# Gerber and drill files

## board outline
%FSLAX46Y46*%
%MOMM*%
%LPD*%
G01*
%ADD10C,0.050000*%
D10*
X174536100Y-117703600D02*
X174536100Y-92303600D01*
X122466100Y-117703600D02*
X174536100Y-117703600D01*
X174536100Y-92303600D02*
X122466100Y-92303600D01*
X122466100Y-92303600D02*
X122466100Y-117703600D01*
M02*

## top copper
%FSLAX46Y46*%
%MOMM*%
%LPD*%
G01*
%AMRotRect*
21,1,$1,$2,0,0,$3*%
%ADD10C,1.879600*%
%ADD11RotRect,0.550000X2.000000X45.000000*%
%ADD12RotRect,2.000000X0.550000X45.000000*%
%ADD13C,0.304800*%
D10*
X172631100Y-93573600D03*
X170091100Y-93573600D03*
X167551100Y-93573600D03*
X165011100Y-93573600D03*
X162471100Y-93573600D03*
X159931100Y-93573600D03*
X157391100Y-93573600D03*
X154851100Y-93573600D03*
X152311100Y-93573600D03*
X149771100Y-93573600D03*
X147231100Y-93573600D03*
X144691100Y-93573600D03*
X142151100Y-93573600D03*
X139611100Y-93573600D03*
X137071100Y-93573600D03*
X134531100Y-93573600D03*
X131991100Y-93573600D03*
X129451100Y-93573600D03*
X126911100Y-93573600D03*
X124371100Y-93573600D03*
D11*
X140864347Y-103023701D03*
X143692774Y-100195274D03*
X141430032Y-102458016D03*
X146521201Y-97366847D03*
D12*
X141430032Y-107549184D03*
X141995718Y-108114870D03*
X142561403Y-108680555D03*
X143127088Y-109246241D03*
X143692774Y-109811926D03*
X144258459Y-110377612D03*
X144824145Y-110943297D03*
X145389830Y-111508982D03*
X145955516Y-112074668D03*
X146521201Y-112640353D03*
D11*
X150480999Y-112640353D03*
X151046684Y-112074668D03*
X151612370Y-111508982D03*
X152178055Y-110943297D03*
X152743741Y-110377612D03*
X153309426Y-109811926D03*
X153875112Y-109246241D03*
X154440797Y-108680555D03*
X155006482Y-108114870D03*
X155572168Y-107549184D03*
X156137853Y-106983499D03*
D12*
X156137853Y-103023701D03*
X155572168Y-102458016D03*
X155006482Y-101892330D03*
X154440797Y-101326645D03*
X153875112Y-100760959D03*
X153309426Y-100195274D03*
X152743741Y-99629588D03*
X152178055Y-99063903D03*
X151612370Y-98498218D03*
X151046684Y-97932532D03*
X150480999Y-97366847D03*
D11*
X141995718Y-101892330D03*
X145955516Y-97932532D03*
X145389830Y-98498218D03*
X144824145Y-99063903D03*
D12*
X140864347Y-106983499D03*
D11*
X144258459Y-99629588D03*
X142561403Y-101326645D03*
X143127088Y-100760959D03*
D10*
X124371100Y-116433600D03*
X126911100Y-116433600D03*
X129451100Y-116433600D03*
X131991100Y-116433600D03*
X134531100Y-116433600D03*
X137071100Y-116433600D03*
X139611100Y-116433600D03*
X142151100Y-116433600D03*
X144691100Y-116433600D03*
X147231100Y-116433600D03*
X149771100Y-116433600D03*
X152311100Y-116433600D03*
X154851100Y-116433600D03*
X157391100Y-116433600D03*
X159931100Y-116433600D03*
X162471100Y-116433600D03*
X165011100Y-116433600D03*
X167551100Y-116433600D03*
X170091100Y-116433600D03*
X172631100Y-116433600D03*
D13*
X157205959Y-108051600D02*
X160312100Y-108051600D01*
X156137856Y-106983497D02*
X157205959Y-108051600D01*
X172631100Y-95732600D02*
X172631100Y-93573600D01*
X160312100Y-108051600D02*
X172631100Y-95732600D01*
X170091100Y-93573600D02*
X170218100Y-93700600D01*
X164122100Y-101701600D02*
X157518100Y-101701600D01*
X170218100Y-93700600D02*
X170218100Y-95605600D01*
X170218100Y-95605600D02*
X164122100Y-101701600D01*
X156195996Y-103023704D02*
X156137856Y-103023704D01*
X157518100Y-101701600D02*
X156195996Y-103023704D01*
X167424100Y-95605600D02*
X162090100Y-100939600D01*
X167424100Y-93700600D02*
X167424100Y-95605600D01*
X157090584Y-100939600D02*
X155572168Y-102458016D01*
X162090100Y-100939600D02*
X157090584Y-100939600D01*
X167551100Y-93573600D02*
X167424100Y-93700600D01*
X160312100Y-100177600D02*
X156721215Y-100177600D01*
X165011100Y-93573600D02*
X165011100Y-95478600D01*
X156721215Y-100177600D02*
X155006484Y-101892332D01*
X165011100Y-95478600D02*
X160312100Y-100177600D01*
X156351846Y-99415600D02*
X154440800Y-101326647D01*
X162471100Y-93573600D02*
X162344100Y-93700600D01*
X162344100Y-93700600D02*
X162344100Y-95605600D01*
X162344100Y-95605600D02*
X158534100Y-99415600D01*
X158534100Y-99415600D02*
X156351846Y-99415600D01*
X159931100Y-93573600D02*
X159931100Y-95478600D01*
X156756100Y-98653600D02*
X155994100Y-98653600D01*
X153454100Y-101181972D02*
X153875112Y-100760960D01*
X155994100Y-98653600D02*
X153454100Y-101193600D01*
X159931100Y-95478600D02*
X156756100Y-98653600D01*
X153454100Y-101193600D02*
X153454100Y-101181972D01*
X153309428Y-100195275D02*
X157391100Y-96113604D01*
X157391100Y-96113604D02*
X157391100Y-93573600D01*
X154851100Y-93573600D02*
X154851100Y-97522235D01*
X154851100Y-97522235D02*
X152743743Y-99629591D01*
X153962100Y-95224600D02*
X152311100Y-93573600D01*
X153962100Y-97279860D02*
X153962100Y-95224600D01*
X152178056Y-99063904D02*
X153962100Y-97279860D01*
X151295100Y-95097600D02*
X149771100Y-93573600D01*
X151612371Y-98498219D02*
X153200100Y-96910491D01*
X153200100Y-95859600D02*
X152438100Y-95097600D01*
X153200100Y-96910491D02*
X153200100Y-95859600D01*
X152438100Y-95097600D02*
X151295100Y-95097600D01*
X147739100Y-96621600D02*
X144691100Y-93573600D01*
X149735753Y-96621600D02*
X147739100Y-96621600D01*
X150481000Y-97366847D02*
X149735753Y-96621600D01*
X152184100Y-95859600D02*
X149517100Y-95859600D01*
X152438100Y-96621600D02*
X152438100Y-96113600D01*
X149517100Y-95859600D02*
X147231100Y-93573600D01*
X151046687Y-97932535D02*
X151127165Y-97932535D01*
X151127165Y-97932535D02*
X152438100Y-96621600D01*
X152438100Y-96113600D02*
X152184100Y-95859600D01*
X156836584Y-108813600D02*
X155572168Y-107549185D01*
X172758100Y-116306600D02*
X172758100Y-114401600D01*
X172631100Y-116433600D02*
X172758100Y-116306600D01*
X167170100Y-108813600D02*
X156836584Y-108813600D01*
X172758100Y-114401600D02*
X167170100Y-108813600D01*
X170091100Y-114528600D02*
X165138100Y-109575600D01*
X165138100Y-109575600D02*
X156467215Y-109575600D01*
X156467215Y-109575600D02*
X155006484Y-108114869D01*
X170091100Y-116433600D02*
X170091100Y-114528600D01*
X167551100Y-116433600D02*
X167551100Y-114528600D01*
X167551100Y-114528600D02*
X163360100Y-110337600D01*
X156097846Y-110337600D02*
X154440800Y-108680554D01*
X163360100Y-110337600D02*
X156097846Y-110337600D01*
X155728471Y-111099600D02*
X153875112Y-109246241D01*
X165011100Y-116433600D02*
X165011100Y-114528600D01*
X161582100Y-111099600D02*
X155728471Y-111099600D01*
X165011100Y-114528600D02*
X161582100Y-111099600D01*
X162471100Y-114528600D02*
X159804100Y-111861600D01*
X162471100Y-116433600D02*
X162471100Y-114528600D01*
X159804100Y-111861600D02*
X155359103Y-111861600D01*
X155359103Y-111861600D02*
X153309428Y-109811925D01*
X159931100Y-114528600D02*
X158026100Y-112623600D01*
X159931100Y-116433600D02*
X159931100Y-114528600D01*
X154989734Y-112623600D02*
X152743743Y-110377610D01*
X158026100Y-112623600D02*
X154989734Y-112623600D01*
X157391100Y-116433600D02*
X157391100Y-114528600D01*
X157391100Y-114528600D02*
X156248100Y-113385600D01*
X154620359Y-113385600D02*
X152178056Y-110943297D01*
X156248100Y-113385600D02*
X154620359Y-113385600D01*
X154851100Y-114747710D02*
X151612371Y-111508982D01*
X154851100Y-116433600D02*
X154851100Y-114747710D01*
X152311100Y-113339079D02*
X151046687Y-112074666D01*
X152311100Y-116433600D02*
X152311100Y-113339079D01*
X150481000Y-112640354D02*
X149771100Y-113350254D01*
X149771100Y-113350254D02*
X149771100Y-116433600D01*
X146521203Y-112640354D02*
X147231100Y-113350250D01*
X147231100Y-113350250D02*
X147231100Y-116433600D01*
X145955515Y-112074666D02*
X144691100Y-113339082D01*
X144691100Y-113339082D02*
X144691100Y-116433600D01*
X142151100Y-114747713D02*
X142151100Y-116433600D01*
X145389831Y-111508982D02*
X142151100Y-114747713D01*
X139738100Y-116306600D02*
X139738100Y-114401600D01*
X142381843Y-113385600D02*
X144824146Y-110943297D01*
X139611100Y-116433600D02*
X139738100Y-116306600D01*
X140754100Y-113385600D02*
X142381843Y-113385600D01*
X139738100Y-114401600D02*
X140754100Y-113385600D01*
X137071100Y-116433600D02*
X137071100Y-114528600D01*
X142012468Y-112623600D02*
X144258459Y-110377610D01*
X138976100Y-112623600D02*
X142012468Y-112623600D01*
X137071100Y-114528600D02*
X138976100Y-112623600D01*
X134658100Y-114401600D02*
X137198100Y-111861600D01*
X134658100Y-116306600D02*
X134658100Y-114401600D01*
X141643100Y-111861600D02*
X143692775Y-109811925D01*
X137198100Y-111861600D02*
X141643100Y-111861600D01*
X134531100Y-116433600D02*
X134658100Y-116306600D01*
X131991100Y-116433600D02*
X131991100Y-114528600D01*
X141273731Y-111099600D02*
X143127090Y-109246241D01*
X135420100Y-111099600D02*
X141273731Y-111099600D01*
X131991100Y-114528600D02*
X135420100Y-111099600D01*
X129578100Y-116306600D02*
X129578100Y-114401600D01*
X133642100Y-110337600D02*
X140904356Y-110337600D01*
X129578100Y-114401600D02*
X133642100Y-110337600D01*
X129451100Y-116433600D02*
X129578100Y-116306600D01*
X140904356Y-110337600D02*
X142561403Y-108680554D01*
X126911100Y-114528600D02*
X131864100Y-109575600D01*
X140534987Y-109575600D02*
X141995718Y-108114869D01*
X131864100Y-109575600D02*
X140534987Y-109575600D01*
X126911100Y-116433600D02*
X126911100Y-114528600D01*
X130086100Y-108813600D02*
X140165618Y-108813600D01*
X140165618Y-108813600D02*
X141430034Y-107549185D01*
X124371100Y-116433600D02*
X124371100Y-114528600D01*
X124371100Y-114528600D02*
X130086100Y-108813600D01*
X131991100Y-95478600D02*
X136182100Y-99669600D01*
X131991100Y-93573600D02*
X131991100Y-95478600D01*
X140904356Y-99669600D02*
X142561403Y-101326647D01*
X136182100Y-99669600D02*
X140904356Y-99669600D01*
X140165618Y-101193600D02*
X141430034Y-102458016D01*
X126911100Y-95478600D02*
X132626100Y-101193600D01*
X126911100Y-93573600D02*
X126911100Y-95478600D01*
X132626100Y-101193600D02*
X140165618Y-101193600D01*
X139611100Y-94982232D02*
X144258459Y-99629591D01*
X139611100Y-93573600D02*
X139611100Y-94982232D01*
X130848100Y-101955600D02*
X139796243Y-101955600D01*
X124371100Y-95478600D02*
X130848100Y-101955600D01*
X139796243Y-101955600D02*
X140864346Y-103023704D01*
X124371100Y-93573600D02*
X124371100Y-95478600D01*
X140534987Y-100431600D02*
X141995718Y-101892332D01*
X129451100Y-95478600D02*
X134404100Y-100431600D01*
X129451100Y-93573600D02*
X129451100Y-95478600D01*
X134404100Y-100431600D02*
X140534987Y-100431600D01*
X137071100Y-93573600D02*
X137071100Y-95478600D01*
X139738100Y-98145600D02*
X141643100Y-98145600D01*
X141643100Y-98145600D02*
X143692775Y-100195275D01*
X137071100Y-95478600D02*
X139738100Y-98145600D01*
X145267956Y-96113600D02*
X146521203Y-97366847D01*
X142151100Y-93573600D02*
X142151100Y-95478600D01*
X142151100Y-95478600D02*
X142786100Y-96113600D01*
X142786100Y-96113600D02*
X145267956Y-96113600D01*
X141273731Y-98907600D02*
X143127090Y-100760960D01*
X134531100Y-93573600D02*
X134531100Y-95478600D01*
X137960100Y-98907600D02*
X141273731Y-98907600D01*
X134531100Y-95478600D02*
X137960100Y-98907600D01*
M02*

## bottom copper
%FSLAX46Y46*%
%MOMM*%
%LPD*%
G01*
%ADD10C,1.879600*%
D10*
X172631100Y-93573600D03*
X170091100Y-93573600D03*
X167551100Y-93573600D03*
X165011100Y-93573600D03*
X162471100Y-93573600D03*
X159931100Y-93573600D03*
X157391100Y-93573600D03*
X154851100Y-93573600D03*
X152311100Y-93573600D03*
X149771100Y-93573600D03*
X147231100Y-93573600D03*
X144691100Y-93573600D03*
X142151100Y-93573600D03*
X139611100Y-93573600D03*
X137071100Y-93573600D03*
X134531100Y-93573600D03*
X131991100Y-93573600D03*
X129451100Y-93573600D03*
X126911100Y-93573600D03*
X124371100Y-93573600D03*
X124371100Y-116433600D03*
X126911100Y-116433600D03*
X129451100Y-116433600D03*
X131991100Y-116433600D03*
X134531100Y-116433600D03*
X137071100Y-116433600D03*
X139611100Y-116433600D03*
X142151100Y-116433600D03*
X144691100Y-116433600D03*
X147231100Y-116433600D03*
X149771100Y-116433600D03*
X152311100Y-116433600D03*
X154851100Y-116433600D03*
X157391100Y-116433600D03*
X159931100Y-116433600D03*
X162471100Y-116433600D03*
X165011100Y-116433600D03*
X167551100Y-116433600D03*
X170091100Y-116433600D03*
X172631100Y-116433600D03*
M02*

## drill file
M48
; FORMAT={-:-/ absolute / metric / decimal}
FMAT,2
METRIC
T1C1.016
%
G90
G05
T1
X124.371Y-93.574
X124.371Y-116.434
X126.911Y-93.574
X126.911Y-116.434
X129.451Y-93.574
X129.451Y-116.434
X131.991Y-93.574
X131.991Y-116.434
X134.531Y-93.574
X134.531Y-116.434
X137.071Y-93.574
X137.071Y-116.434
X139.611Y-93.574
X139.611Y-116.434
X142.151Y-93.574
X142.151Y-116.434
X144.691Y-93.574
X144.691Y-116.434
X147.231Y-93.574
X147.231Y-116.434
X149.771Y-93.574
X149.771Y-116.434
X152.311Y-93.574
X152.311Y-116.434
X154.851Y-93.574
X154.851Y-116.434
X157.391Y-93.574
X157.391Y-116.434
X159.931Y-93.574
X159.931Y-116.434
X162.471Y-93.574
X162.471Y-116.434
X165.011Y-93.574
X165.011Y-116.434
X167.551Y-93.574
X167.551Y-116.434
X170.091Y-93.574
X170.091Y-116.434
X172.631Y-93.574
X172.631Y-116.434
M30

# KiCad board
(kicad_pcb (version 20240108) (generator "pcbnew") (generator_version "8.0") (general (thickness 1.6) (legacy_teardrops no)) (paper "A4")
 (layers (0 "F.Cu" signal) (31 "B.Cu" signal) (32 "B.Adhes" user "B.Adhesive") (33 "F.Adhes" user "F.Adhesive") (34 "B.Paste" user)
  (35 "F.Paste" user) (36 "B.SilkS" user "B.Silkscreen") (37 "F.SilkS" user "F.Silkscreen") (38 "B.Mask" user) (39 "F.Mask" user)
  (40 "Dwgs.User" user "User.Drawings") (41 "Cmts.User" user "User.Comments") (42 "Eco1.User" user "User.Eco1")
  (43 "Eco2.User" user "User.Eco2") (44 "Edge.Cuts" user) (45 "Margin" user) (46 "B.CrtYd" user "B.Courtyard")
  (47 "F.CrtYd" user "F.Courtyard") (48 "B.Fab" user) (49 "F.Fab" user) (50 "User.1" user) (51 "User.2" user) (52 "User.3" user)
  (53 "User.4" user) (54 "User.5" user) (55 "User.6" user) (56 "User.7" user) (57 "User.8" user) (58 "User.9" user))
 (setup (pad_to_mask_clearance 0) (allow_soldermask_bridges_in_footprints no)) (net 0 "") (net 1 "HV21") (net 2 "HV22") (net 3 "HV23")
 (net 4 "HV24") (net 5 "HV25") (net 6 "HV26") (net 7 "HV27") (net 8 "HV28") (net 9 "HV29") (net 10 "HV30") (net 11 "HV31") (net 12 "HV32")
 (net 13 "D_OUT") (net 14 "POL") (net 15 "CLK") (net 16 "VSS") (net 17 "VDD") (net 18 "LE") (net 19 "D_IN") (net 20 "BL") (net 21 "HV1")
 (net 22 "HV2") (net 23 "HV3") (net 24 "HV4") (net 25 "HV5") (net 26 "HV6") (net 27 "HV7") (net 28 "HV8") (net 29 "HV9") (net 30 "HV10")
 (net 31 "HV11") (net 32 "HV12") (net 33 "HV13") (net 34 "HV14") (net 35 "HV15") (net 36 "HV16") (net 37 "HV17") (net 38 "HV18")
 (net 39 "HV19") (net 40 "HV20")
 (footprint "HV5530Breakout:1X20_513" (layer "F.Cu") (at 172.6311 93.5736 180)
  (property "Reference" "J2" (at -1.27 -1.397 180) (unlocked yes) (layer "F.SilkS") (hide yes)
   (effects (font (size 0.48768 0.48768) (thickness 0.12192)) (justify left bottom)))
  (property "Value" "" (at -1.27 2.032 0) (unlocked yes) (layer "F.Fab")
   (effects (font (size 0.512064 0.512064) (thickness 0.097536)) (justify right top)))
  (pad "1" thru_hole circle (at 0 0 270) (size 1.8796 1.8796) (drill 1.016) (layers "*.Cu" "*.Mask") (remove_unused_layers no)
   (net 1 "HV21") (solder_mask_margin 0.1016) (thermal_bridge_angle 0))
  (pad "2" thru_hole circle (at 2.54 0 270) (size 1.8796 1.8796) (drill 1.016) (layers "*.Cu" "*.Mask") (remove_unused_layers no)
   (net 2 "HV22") (solder_mask_margin 0.1016) (thermal_bridge_angle 0))
  (pad "3" thru_hole circle (at 5.08 0 270) (size 1.8796 1.8796) (drill 1.016) (layers "*.Cu" "*.Mask") (remove_unused_layers no)
   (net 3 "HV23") (solder_mask_margin 0.1016) (thermal_bridge_angle 0))
  (pad "4" thru_hole circle (at 7.62 0 270) (size 1.8796 1.8796) (drill 1.016) (layers "*.Cu" "*.Mask") (remove_unused_layers no)
   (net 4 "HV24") (solder_mask_margin 0.1016) (thermal_bridge_angle 0))
  (pad "5" thru_hole circle (at 10.16 0 270) (size 1.8796 1.8796) (drill 1.016) (layers "*.Cu" "*.Mask") (remove_unused_layers no)
   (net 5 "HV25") (solder_mask_margin 0.1016) (thermal_bridge_angle 0))
  (pad "6" thru_hole circle (at 12.7 0 270) (size 1.8796 1.8796) (drill 1.016) (layers "*.Cu" "*.Mask") (remove_unused_layers no)
   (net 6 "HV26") (solder_mask_margin 0.1016) (thermal_bridge_angle 0))
  (pad "7" thru_hole circle (at 15.24 0 270) (size 1.8796 1.8796) (drill 1.016) (layers "*.Cu" "*.Mask") (remove_unused_layers no)
   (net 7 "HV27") (solder_mask_margin 0.1016) (thermal_bridge_angle 0))
  (pad "8" thru_hole circle (at 17.78 0 270) (size 1.8796 1.8796) (drill 1.016) (layers "*.Cu" "*.Mask") (remove_unused_layers no)
   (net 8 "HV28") (solder_mask_margin 0.1016) (thermal_bridge_angle 0))
  (pad "9" thru_hole circle (at 20.32 0 270) (size 1.8796 1.8796) (drill 1.016) (layers "*.Cu" "*.Mask") (remove_unused_layers no)
   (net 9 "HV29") (solder_mask_margin 0.1016) (thermal_bridge_angle 0))
  (pad "10" thru_hole circle (at 22.86 0 270) (size 1.8796 1.8796) (drill 1.016) (layers "*.Cu" "*.Mask") (remove_unused_layers no)
   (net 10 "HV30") (solder_mask_margin 0.1016) (thermal_bridge_angle 0))
  (pad "11" thru_hole circle (at 25.4 0 270) (size 1.8796 1.8796) (drill 1.016) (layers "*.Cu" "*.Mask") (remove_unused_layers no)
   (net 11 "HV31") (solder_mask_margin 0.1016) (thermal_bridge_angle 0))
  (pad "12" thru_hole circle (at 27.94 0 270) (size 1.8796 1.8796) (drill 1.016) (layers "*.Cu" "*.Mask") (remove_unused_layers no)
   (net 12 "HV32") (solder_mask_margin 0.1016) (thermal_bridge_angle 0))
  (pad "13" thru_hole circle (at 30.48 0 270) (size 1.8796 1.8796) (drill 1.016) (layers "*.Cu" "*.Mask") (remove_unused_layers no)
   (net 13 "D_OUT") (solder_mask_margin 0.1016) (thermal_bridge_angle 0))
  (pad "14" thru_hole circle (at 33.02 0 270) (size 1.8796 1.8796) (drill 1.016) (layers "*.Cu" "*.Mask") (remove_unused_layers no)
   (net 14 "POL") (solder_mask_margin 0.1016) (thermal_bridge_angle 0))
  (pad "15" thru_hole circle (at 35.56 0 270) (size 1.8796 1.8796) (drill 1.016) (layers "*.Cu" "*.Mask") (remove_unused_layers no)
   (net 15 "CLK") (solder_mask_margin 0.1016) (thermal_bridge_angle 0))
  (pad "16" thru_hole circle (at 38.1 0 270) (size 1.8796 1.8796) (drill 1.016) (layers "*.Cu" "*.Mask") (remove_unused_layers no)
   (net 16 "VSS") (solder_mask_margin 0.1016) (thermal_bridge_angle 0))
  (pad "17" thru_hole circle (at 40.64 0 270) (size 1.8796 1.8796) (drill 1.016) (layers "*.Cu" "*.Mask") (remove_unused_layers no)
   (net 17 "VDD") (solder_mask_margin 0.1016) (thermal_bridge_angle 0))
  (pad "18" thru_hole circle (at 43.18 0 270) (size 1.8796 1.8796) (drill 1.016) (layers "*.Cu" "*.Mask") (remove_unused_layers no)
   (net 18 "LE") (solder_mask_margin 0.1016) (thermal_bridge_angle 0))
  (pad "19" thru_hole circle (at 45.72 0 270) (size 1.8796 1.8796) (drill 1.016) (layers "*.Cu" "*.Mask") (remove_unused_layers no)
   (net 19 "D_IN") (solder_mask_margin 0.1016) (thermal_bridge_angle 0))
  (pad "20" thru_hole circle (at 48.26 0 270) (size 1.8796 1.8796) (drill 1.016) (layers "*.Cu" "*.Mask") (remove_unused_layers no)
   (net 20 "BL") (solder_mask_margin 0.1016) (thermal_bridge_angle 0)))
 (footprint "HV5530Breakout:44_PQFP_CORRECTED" (layer "F.Cu") (at 148.5011 105.0036 45)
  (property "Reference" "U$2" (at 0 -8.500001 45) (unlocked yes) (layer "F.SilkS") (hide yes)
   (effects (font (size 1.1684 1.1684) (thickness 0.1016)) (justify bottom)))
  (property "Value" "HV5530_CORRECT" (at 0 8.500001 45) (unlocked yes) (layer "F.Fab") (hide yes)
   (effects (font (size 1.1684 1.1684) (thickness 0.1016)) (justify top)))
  (pad "BL" smd rect (at -4 -6.8 45) (size 0.55 2) (layers "F.Cu" "F.Paste" "F.Mask") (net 20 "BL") (solder_mask_margin 0.1016)
   (thermal_bridge_angle 0))
  (pad "CLK" smd rect (at 0 -6.8 45) (size 0.55 2) (layers "F.Cu" "F.Paste" "F.Mask") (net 15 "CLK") (solder_mask_margin 0.1016)
   (thermal_bridge_angle 0))
  (pad "DIN" smd rect (at -3.2 -6.8 45) (size 0.55 2) (layers "F.Cu" "F.Paste" "F.Mask") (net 19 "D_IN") (solder_mask_margin 0.1016)
   (thermal_bridge_angle 0))
  (pad "DOUT" smd rect (at 4 -6.8 45) (size 0.55 2) (layers "F.Cu" "F.Paste" "F.Mask") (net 13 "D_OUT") (solder_mask_margin 0.1016)
   (thermal_bridge_angle 0))
  (pad "HV1" smd rect (at -6.8 -3.2 45) (size 2 0.55) (layers "F.Cu" "F.Paste" "F.Mask") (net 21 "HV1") (solder_mask_margin 0.1016)
   (thermal_bridge_angle 0))
  (pad "HV2" smd rect (at -6.8 -2.4 45) (size 2 0.55) (layers "F.Cu" "F.Paste" "F.Mask") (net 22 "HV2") (solder_mask_margin 0.1016)
   (thermal_bridge_angle 0))
  (pad "HV3" smd rect (at -6.8 -1.6 45) (size 2 0.55) (layers "F.Cu" "F.Paste" "F.Mask") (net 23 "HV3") (solder_mask_margin 0.1016)
   (thermal_bridge_angle 0))
  (pad "HV4" smd rect (at -6.800001 -0.8 45) (size 2 0.55) (layers "F.Cu" "F.Paste" "F.Mask") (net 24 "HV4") (solder_mask_margin 0.1016)
   (thermal_bridge_angle 0))
  (pad "HV5" smd rect (at -6.8 0 45) (size 2 0.55) (layers "F.Cu" "F.Paste" "F.Mask") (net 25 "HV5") (solder_mask_margin 0.1016)
   (thermal_bridge_angle 0))
  (pad "HV6" smd rect (at -6.800001 0.8 45) (size 2 0.55) (layers "F.Cu" "F.Paste" "F.Mask") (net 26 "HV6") (solder_mask_margin 0.1016)
   (thermal_bridge_angle 0))
  (pad "HV7" smd rect (at -6.8 1.6 45) (size 2 0.55) (layers "F.Cu" "F.Paste" "F.Mask") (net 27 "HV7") (solder_mask_margin 0.1016)
   (thermal_bridge_angle 0))
  (pad "HV8" smd rect (at -6.8 2.4 45) (size 2 0.55) (layers "F.Cu" "F.Paste" "F.Mask") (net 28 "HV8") (solder_mask_margin 0.1016)
   (thermal_bridge_angle 0))
  (pad "HV9" smd rect (at -6.8 3.2 45) (size 2 0.55) (layers "F.Cu" "F.Paste" "F.Mask") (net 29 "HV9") (solder_mask_margin 0.1016)
   (thermal_bridge_angle 0))
  (pad "HV10" smd rect (at -6.8 4 45) (size 2 0.55) (layers "F.Cu" "F.Paste" "F.Mask") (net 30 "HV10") (solder_mask_margin 0.1016)
   (thermal_bridge_angle 0))
  (pad "HV11" smd rect (at -4 6.8 45) (size 0.55 2) (layers "F.Cu" "F.Paste" "F.Mask") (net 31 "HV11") (solder_mask_margin 0.1016)
   (thermal_bridge_angle 0))
  (pad "HV12" smd rect (at -3.2 6.8 45) (size 0.55 2) (layers "F.Cu" "F.Paste" "F.Mask") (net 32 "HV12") (solder_mask_margin 0.1016)
   (thermal_bridge_angle 0))
  (pad "HV13" smd rect (at -2.4 6.8 45) (size 0.55 2) (layers "F.Cu" "F.Paste" "F.Mask") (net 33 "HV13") (solder_mask_margin 0.1016)
   (thermal_bridge_angle 0))
  (pad "HV14" smd rect (at -1.6 6.8 45) (size 0.55 2) (layers "F.Cu" "F.Paste" "F.Mask") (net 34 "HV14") (solder_mask_margin 0.1016)
   (thermal_bridge_angle 0))
  (pad "HV15" smd rect (at -0.8 6.800001 45) (size 0.55 2) (layers "F.Cu" "F.Paste" "F.Mask") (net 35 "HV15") (solder_mask_margin 0.1016)
   (thermal_bridge_angle 0))
  (pad "HV16" smd rect (at 0 6.8 45) (size 0.55 2) (layers "F.Cu" "F.Paste" "F.Mask") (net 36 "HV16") (solder_mask_margin 0.1016)
   (thermal_bridge_angle 0))
  (pad "HV17" smd rect (at 0.8 6.800001 45) (size 0.55 2) (layers "F.Cu" "F.Paste" "F.Mask") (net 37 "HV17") (solder_mask_margin 0.1016)
   (thermal_bridge_angle 0))
  (pad "HV18" smd rect (at 1.6 6.8 45) (size 0.55 2) (layers "F.Cu" "F.Paste" "F.Mask") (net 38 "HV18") (solder_mask_margin 0.1016)
   (thermal_bridge_angle 0))
  (pad "HV19" smd rect (at 2.4 6.8 45) (size 0.55 2) (layers "F.Cu" "F.Paste" "F.Mask") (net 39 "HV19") (solder_mask_margin 0.1016)
   (thermal_bridge_angle 0))
  (pad "HV20" smd rect (at 3.2 6.8 45) (size 0.55 2) (layers "F.Cu" "F.Paste" "F.Mask") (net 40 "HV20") (solder_mask_margin 0.1016)
   (thermal_bridge_angle 0))
  (pad "HV21" smd rect (at 4 6.8 45) (size 0.55 2) (layers "F.Cu" "F.Paste" "F.Mask") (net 1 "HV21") (solder_mask_margin 0.1016)
   (thermal_bridge_angle 0))
  (pad "HV22" smd rect (at 6.8 4 45) (size 2 0.55) (layers "F.Cu" "F.Paste" "F.Mask") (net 2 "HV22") (solder_mask_margin 0.1016)
   (thermal_bridge_angle 0))
  (pad "HV23" smd rect (at 6.8 3.2 45) (size 2 0.55) (layers "F.Cu" "F.Paste" "F.Mask") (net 3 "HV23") (solder_mask_margin 0.1016)
   (thermal_bridge_angle 0))
  (pad "HV24" smd rect (at 6.8 2.4 45) (size 2 0.55) (layers "F.Cu" "F.Paste" "F.Mask") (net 4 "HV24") (solder_mask_margin 0.1016)
   (thermal_bridge_angle 0))
  (pad "HV25" smd rect (at 6.8 1.6 45) (size 2 0.55) (layers "F.Cu" "F.Paste" "F.Mask") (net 5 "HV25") (solder_mask_margin 0.1016)
   (thermal_bridge_angle 0))
  (pad "HV26" smd rect (at 6.800001 0.8 45) (size 2 0.55) (layers "F.Cu" "F.Paste" "F.Mask") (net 6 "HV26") (solder_mask_margin 0.1016)
   (thermal_bridge_angle 0))
  (pad "HV27" smd rect (at 6.8 0 45) (size 2 0.55) (layers "F.Cu" "F.Paste" "F.Mask") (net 7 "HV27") (solder_mask_margin 0.1016)
   (thermal_bridge_angle 0))
  (pad "HV28" smd rect (at 6.800001 -0.8 45) (size 2 0.55) (layers "F.Cu" "F.Paste" "F.Mask") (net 8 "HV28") (solder_mask_margin 0.1016)
   (thermal_bridge_angle 0))
  (pad "HV29" smd rect (at 6.8 -1.6 45) (size 2 0.55) (layers "F.Cu" "F.Paste" "F.Mask") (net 9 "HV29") (solder_mask_margin 0.1016)
   (thermal_bridge_angle 0))
  (pad "HV30" smd rect (at 6.8 -2.4 45) (size 2 0.55) (layers "F.Cu" "F.Paste" "F.Mask") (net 10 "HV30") (solder_mask_margin 0.1016)
   (thermal_bridge_angle 0))
  (pad "HV31" smd rect (at 6.8 -3.2 45) (size 2 0.55) (layers "F.Cu" "F.Paste" "F.Mask") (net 11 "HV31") (solder_mask_margin 0.1016)
   (thermal_bridge_angle 0))
  (pad "HV32" smd rect (at 6.8 -4 45) (size 2 0.55) (layers "F.Cu" "F.Paste" "F.Mask") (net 12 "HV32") (solder_mask_margin 0.1016)
   (thermal_bridge_angle 0))
  (pad "LE" smd rect (at -2.4 -6.8 45) (size 0.55 2) (layers "F.Cu" "F.Paste" "F.Mask") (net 18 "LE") (solder_mask_margin 0.1016)
   (thermal_bridge_angle 0))
  (pad "NC@1" smd rect (at 3.2 -6.8 45) (size 0.55 2) (layers "F.Cu" "F.Paste" "F.Mask") (solder_mask_margin 0.1016)
   (thermal_bridge_angle 0))
  (pad "NC@2" smd rect (at 2.4 -6.8 45) (size 0.55 2) (layers "F.Cu" "F.Paste" "F.Mask") (solder_mask_margin 0.1016)
   (thermal_bridge_angle 0))
  (pad "NC@3" smd rect (at 1.6 -6.8 45) (size 0.55 2) (layers "F.Cu" "F.Paste" "F.Mask") (solder_mask_margin 0.1016)
   (thermal_bridge_angle 0))
  (pad "NC@4" smd rect (at -6.8 -4 45) (size 2 0.55) (layers "F.Cu" "F.Paste" "F.Mask") (solder_mask_margin 0.1016) (thermal_bridge_angle 0))
  (pad "POL" smd rect (at 0.8 -6.800001 45) (size 0.55 2) (layers "F.Cu" "F.Paste" "F.Mask") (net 14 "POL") (solder_mask_margin 0.1016)
   (thermal_bridge_angle 0))
  (pad "VDD" smd rect (at -1.6 -6.8 45) (size 0.55 2) (layers "F.Cu" "F.Paste" "F.Mask") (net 17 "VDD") (solder_mask_margin 0.1016)
   (thermal_bridge_angle 0))
  (pad "VSS" smd rect (at -0.8 -6.800001 45) (size 0.55 2) (layers "F.Cu" "F.Paste" "F.Mask") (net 16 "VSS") (solder_mask_margin 0.1016)
   (thermal_bridge_angle 0)))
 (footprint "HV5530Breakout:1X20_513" (layer "F.Cu") (at 124.3711 116.4336)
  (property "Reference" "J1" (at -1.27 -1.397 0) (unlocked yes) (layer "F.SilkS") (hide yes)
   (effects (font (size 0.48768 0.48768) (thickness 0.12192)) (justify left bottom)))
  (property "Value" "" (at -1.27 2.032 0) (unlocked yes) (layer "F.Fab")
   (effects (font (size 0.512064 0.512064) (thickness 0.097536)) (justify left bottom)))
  (pad "1" thru_hole circle (at 0 0 90) (size 1.8796 1.8796) (drill 1.016) (layers "*.Cu" "*.Mask") (remove_unused_layers no) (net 21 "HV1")
   (solder_mask_margin 0.1016) (thermal_bridge_angle 0))
  (pad "2" thru_hole circle (at 2.54 0 90) (size 1.8796 1.8796) (drill 1.016) (layers "*.Cu" "*.Mask") (remove_unused_layers no)
   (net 22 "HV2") (solder_mask_margin 0.1016) (thermal_bridge_angle 0))
  (pad "3" thru_hole circle (at 5.08 0 90) (size 1.8796 1.8796) (drill 1.016) (layers "*.Cu" "*.Mask") (remove_unused_layers no)
   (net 23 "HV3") (solder_mask_margin 0.1016) (thermal_bridge_angle 0))
  (pad "4" thru_hole circle (at 7.62 0 90) (size 1.8796 1.8796) (drill 1.016) (layers "*.Cu" "*.Mask") (remove_unused_layers no)
   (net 24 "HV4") (solder_mask_margin 0.1016) (thermal_bridge_angle 0))
  (pad "5" thru_hole circle (at 10.16 0 90) (size 1.8796 1.8796) (drill 1.016) (layers "*.Cu" "*.Mask") (remove_unused_layers no)
   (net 25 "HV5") (solder_mask_margin 0.1016) (thermal_bridge_angle 0))
  (pad "6" thru_hole circle (at 12.7 0 90) (size 1.8796 1.8796) (drill 1.016) (layers "*.Cu" "*.Mask") (remove_unused_layers no)
   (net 26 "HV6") (solder_mask_margin 0.1016) (thermal_bridge_angle 0))
  (pad "7" thru_hole circle (at 15.24 0 90) (size 1.8796 1.8796) (drill 1.016) (layers "*.Cu" "*.Mask") (remove_unused_layers no)
   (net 27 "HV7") (solder_mask_margin 0.1016) (thermal_bridge_angle 0))
  (pad "8" thru_hole circle (at 17.78 0 90) (size 1.8796 1.8796) (drill 1.016) (layers "*.Cu" "*.Mask") (remove_unused_layers no)
   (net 28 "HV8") (solder_mask_margin 0.1016) (thermal_bridge_angle 0))
  (pad "9" thru_hole circle (at 20.32 0 90) (size 1.8796 1.8796) (drill 1.016) (layers "*.Cu" "*.Mask") (remove_unused_layers no)
   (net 29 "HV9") (solder_mask_margin 0.1016) (thermal_bridge_angle 0))
  (pad "10" thru_hole circle (at 22.86 0 90) (size 1.8796 1.8796) (drill 1.016) (layers "*.Cu" "*.Mask") (remove_unused_layers no)
   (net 30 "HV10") (solder_mask_margin 0.1016) (thermal_bridge_angle 0))
  (pad "11" thru_hole circle (at 25.4 0 90) (size 1.8796 1.8796) (drill 1.016) (layers "*.Cu" "*.Mask") (remove_unused_layers no)
   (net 31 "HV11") (solder_mask_margin 0.1016) (thermal_bridge_angle 0))
  (pad "12" thru_hole circle (at 27.94 0 90) (size 1.8796 1.8796) (drill 1.016) (layers "*.Cu" "*.Mask") (remove_unused_layers no)
   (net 32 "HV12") (solder_mask_margin 0.1016) (thermal_bridge_angle 0))
  (pad "13" thru_hole circle (at 30.48 0 90) (size 1.8796 1.8796) (drill 1.016) (layers "*.Cu" "*.Mask") (remove_unused_layers no)
   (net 33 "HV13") (solder_mask_margin 0.1016) (thermal_bridge_angle 0))
  (pad "14" thru_hole circle (at 33.02 0 90) (size 1.8796 1.8796) (drill 1.016) (layers "*.Cu" "*.Mask") (remove_unused_layers no)
   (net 34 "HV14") (solder_mask_margin 0.1016) (thermal_bridge_angle 0))
  (pad "15" thru_hole circle (at 35.56 0 90) (size 1.8796 1.8796) (drill 1.016) (layers "*.Cu" "*.Mask") (remove_unused_layers no)
   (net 35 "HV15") (solder_mask_margin 0.1016) (thermal_bridge_angle 0))
  (pad "16" thru_hole circle (at 38.1 0 90) (size 1.8796 1.8796) (drill 1.016) (layers "*.Cu" "*.Mask") (remove_unused_layers no)
   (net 36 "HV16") (solder_mask_margin 0.1016) (thermal_bridge_angle 0))
  (pad "17" thru_hole circle (at 40.64 0 90) (size 1.8796 1.8796) (drill 1.016) (layers "*.Cu" "*.Mask") (remove_unused_layers no)
   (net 37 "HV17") (solder_mask_margin 0.1016) (thermal_bridge_angle 0))
  (pad "18" thru_hole circle (at 43.18 0 90) (size 1.8796 1.8796) (drill 1.016) (layers "*.Cu" "*.Mask") (remove_unused_layers no)
   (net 38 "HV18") (solder_mask_margin 0.1016) (thermal_bridge_angle 0))
  (pad "19" thru_hole circle (at 45.72 0 90) (size 1.8796 1.8796) (drill 1.016) (layers "*.Cu" "*.Mask") (remove_unused_layers no)
   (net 39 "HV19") (solder_mask_margin 0.1016) (thermal_bridge_angle 0))
  (pad "20" thru_hole circle (at 48.26 0 90) (size 1.8796 1.8796) (drill 1.016) (layers "*.Cu" "*.Mask") (remove_unused_layers no)
   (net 40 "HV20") (solder_mask_margin 0.1016) (thermal_bridge_angle 0)))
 (gr_line (start 174.5361 117.7036) (end 174.5361 92.3036) (stroke (width 0.05) (type solid)) (layer "Edge.Cuts"))
 (gr_line (start 122.4661 117.7036) (end 174.5361 117.7036) (stroke (width 0.05) (type solid)) (layer "Edge.Cuts"))
 (gr_line (start 174.5361 92.3036) (end 122.4661 92.3036) (stroke (width 0.05) (type solid)) (layer "Edge.Cuts"))
 (gr_line (start 122.4661 92.3036) (end 122.4661 117.7036) (stroke (width 0.05) (type solid)) (layer "Edge.Cuts"))
 (segment (start 157.205959 108.0516) (end 160.3121 108.0516) (width 0.3048) (layer "F.Cu") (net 1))
 (segment (start 156.137856 106.983497) (end 157.205959 108.0516) (width 0.3048) (layer "F.Cu") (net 1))
 (segment (start 172.6311 95.7326) (end 172.6311 93.5736) (width 0.3048) (layer "F.Cu") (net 1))
 (segment (start 160.3121 108.0516) (end 172.6311 95.7326) (width 0.3048) (layer "F.Cu") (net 1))
 (segment (start 170.0911 93.5736) (end 170.2181 93.7006) (width 0.3048) (layer "F.Cu") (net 2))
 (segment (start 164.1221 101.7016) (end 157.5181 101.7016) (width 0.3048) (layer "F.Cu") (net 2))
 (segment (start 170.2181 93.7006) (end 170.2181 95.6056) (width 0.3048) (layer "F.Cu") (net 2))
 (segment (start 170.2181 95.6056) (end 164.1221 101.7016) (width 0.3048) (layer "F.Cu") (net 2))
 (segment (start 156.195996 103.023704) (end 156.137856 103.023704) (width 0.3048) (layer "F.Cu") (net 2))
 (segment (start 157.5181 101.7016) (end 156.195996 103.023704) (width 0.3048) (layer "F.Cu") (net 2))
 (segment (start 167.4241 95.6056) (end 162.0901 100.9396) (width 0.3048) (layer "F.Cu") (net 3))
 (segment (start 167.4241 93.7006) (end 167.4241 95.6056) (width 0.3048) (layer "F.Cu") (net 3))
 (segment (start 157.090584 100.9396) (end 155.572168 102.458016) (width 0.3048) (layer "F.Cu") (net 3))
 (segment (start 162.0901 100.9396) (end 157.090584 100.9396) (width 0.3048) (layer "F.Cu") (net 3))
 (segment (start 167.5511 93.5736) (end 167.4241 93.7006) (width 0.3048) (layer "F.Cu") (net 3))
 (segment (start 160.3121 100.1776) (end 156.721215 100.1776) (width 0.3048) (layer "F.Cu") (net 4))
 (segment (start 165.0111 93.5736) (end 165.0111 95.4786) (width 0.3048) (layer "F.Cu") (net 4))
 (segment (start 156.721215 100.1776) (end 155.006484 101.892332) (width 0.3048) (layer "F.Cu") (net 4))
 (segment (start 165.0111 95.4786) (end 160.3121 100.1776) (width 0.3048) (layer "F.Cu") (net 4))
 (segment (start 156.351846 99.4156) (end 154.4408 101.326647) (width 0.3048) (layer "F.Cu") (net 5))
 (segment (start 162.4711 93.5736) (end 162.3441 93.7006) (width 0.3048) (layer "F.Cu") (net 5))
 (segment (start 162.3441 93.7006) (end 162.3441 95.6056) (width 0.3048) (layer "F.Cu") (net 5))
 (segment (start 162.3441 95.6056) (end 158.5341 99.4156) (width 0.3048) (layer "F.Cu") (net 5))
 (segment (start 158.5341 99.4156) (end 156.351846 99.4156) (width 0.3048) (layer "F.Cu") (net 5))
 (segment (start 159.9311 93.5736) (end 159.9311 95.4786) (width 0.3048) (layer "F.Cu") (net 6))
 (segment (start 156.7561 98.6536) (end 155.9941 98.6536) (width 0.3048) (layer "F.Cu") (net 6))
 (segment (start 153.4541 101.181972) (end 153.875112 100.76096) (width 0.3048) (layer "F.Cu") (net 6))
 (segment (start 155.9941 98.6536) (end 153.4541 101.1936) (width 0.3048) (layer "F.Cu") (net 6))
 (segment (start 159.9311 95.4786) (end 156.7561 98.6536) (width 0.3048) (layer "F.Cu") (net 6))
 (segment (start 153.4541 101.1936) (end 153.4541 101.181972) (width 0.3048) (layer "F.Cu") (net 6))
 (segment (start 153.309428 100.195275) (end 157.3911 96.113604) (width 0.3048) (layer "F.Cu") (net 7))
 (segment (start 157.3911 96.113604) (end 157.3911 93.5736) (width 0.3048) (layer "F.Cu") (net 7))
 (segment (start 154.8511 93.5736) (end 154.8511 97.522235) (width 0.3048) (layer "F.Cu") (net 8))
 (segment (start 154.8511 97.522235) (end 152.743743 99.629591) (width 0.3048) (layer "F.Cu") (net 8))
 (segment (start 153.9621 95.2246) (end 152.3111 93.5736) (width 0.3048) (layer "F.Cu") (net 9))
 (segment (start 153.9621 97.27986) (end 153.9621 95.2246) (width 0.3048) (layer "F.Cu") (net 9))
 (segment (start 152.178056 99.063904) (end 153.9621 97.27986) (width 0.3048) (layer "F.Cu") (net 9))
 (segment (start 151.2951 95.0976) (end 149.7711 93.5736) (width 0.3048) (layer "F.Cu") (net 10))
 (segment (start 151.612371 98.498219) (end 153.2001 96.910491) (width 0.3048) (layer "F.Cu") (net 10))
 (segment (start 153.2001 95.8596) (end 152.4381 95.0976) (width 0.3048) (layer "F.Cu") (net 10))
 (segment (start 153.2001 96.910491) (end 153.2001 95.8596) (width 0.3048) (layer "F.Cu") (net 10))
 (segment (start 152.4381 95.0976) (end 151.2951 95.0976) (width 0.3048) (layer "F.Cu") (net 10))
 (segment (start 147.7391 96.6216) (end 144.6911 93.5736) (width 0.3048) (layer "F.Cu") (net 12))
 (segment (start 149.735753 96.6216) (end 147.7391 96.6216) (width 0.3048) (layer "F.Cu") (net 12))
 (segment (start 150.481 97.366847) (end 149.735753 96.6216) (width 0.3048) (layer "F.Cu") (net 12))
 (segment (start 152.1841 95.8596) (end 149.5171 95.8596) (width 0.3048) (layer "F.Cu") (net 11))
 (segment (start 152.4381 96.6216) (end 152.4381 96.1136) (width 0.3048) (layer "F.Cu") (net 11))
 (segment (start 149.5171 95.8596) (end 147.2311 93.5736) (width 0.3048) (layer "F.Cu") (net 11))
 (segment (start 151.046687 97.932535) (end 151.127165 97.932535) (width 0.3048) (layer "F.Cu") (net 11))
 (segment (start 151.127165 97.932535) (end 152.4381 96.6216) (width 0.3048) (layer "F.Cu") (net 11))
 (segment (start 152.4381 96.1136) (end 152.1841 95.8596) (width 0.3048) (layer "F.Cu") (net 11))
 (segment (start 156.836584 108.8136) (end 155.572168 107.549185) (width 0.3048) (layer "F.Cu") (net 40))
 (segment (start 172.7581 116.3066) (end 172.7581 114.4016) (width 0.3048) (layer "F.Cu") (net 40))
 (segment (start 172.6311 116.4336) (end 172.7581 116.3066) (width 0.3048) (layer "F.Cu") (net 40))
 (segment (start 167.1701 108.8136) (end 156.836584 108.8136) (width 0.3048) (layer "F.Cu") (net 40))
 (segment (start 172.7581 114.4016) (end 167.1701 108.8136) (width 0.3048) (layer "F.Cu") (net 40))
 (segment (start 170.0911 114.5286) (end 165.1381 109.5756) (width 0.3048) (layer "F.Cu") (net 39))
 (segment (start 165.1381 109.5756) (end 156.467215 109.5756) (width 0.3048) (layer "F.Cu") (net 39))
 (segment (start 156.467215 109.5756) (end 155.006484 108.114869) (width 0.3048) (layer "F.Cu") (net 39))
 (segment (start 170.0911 116.4336) (end 170.0911 114.5286) (width 0.3048) (layer "F.Cu") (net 39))
 (segment (start 167.5511 116.4336) (end 167.5511 114.5286) (width 0.3048) (layer "F.Cu") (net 38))
 (segment (start 167.5511 114.5286) (end 163.3601 110.3376) (width 0.3048) (layer "F.Cu") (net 38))
 (segment (start 156.097846 110.3376) (end 154.4408 108.680554) (width 0.3048) (layer "F.Cu") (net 38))
 (segment (start 163.3601 110.3376) (end 156.097846 110.3376) (width 0.3048) (layer "F.Cu") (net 38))
 (segment (start 155.728471 111.0996) (end 153.875112 109.246241) (width 0.3048) (layer "F.Cu") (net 37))
 (segment (start 165.0111 116.4336) (end 165.0111 114.5286) (width 0.3048) (layer "F.Cu") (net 37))
 (segment (start 161.5821 111.0996) (end 155.728471 111.0996) (width 0.3048) (layer "F.Cu") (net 37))
 (segment (start 165.0111 114.5286) (end 161.5821 111.0996) (width 0.3048) (layer "F.Cu") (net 37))
 (segment (start 162.4711 114.5286) (end 159.8041 111.8616) (width 0.3048) (layer "F.Cu") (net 36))
 (segment (start 162.4711 116.4336) (end 162.4711 114.5286) (width 0.3048) (layer "F.Cu") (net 36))
 (segment (start 159.8041 111.8616) (end 155.359103 111.8616) (width 0.3048) (layer "F.Cu") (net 36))
 (segment (start 155.359103 111.8616) (end 153.309428 109.811925) (width 0.3048) (layer "F.Cu") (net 36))
 (segment (start 159.9311 114.5286) (end 158.0261 112.6236) (width 0.3048) (layer "F.Cu") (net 35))
 (segment (start 159.9311 116.4336) (end 159.9311 114.5286) (width 0.3048) (layer "F.Cu") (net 35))
 (segment (start 154.989734 112.6236) (end 152.743743 110.37761) (width 0.3048) (layer "F.Cu") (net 35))
 (segment (start 158.0261 112.6236) (end 154.989734 112.6236) (width 0.3048) (layer "F.Cu") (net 35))
 (segment (start 157.3911 116.4336) (end 157.3911 114.5286) (width 0.3048) (layer "F.Cu") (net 34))
 (segment (start 157.3911 114.5286) (end 156.2481 113.3856) (width 0.3048) (layer "F.Cu") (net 34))
 (segment (start 154.620359 113.3856) (end 152.178056 110.943297) (width 0.3048) (layer "F.Cu") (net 34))
 (segment (start 156.2481 113.3856) (end 154.620359 113.3856) (width 0.3048) (layer "F.Cu") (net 34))
 (segment (start 154.8511 114.74771) (end 151.612371 111.508982) (width 0.3048) (layer "F.Cu") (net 33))
 (segment (start 154.8511 116.4336) (end 154.8511 114.74771) (width 0.3048) (layer "F.Cu") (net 33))
 (segment (start 152.3111 113.339079) (end 151.046687 112.074666) (width 0.3048) (layer "F.Cu") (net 32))
 (segment (start 152.3111 116.4336) (end 152.3111 113.339079) (width 0.3048) (layer "F.Cu") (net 32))
 (segment (start 150.481 112.640354) (end 149.7711 113.350254) (width 0.3048) (layer "F.Cu") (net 31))
 (segment (start 149.7711 113.350254) (end 149.7711 116.4336) (width 0.3048) (layer "F.Cu") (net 31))
 (segment (start 146.521203 112.640354) (end 147.2311 113.35025) (width 0.3048) (layer "F.Cu") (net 30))
 (segment (start 147.2311 113.35025) (end 147.2311 116.4336) (width 0.3048) (layer "F.Cu") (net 30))
 (segment (start 145.955515 112.074666) (end 144.6911 113.339082) (width 0.3048) (layer "F.Cu") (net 29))
 (segment (start 144.6911 113.339082) (end 144.6911 116.4336) (width 0.3048) (layer "F.Cu") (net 29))
 (segment (start 142.1511 114.747713) (end 142.1511 116.4336) (width 0.3048) (layer "F.Cu") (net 28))
 (segment (start 145.389831 111.508982) (end 142.1511 114.747713) (width 0.3048) (layer "F.Cu") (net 28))
 (segment (start 139.7381 116.3066) (end 139.7381 114.4016) (width 0.3048) (layer "F.Cu") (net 27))
 (segment (start 142.381843 113.3856) (end 144.824146 110.943297) (width 0.3048) (layer "F.Cu") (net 27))
 (segment (start 139.6111 116.4336) (end 139.7381 116.3066) (width 0.3048) (layer "F.Cu") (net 27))
 (segment (start 140.7541 113.3856) (end 142.381843 113.3856) (width 0.3048) (layer "F.Cu") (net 27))
 (segment (start 139.7381 114.4016) (end 140.7541 113.3856) (width 0.3048) (layer "F.Cu") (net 27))
 (segment (start 137.0711 116.4336) (end 137.0711 114.5286) (width 0.3048) (layer "F.Cu") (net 26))
 (segment (start 142.012468 112.6236) (end 144.258459 110.37761) (width 0.3048) (layer "F.Cu") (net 26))
 (segment (start 138.9761 112.6236) (end 142.012468 112.6236) (width 0.3048) (layer "F.Cu") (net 26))
 (segment (start 137.0711 114.5286) (end 138.9761 112.6236) (width 0.3048) (layer "F.Cu") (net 26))
 (segment (start 134.6581 114.4016) (end 137.1981 111.8616) (width 0.3048) (layer "F.Cu") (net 25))
 (segment (start 134.6581 116.3066) (end 134.6581 114.4016) (width 0.3048) (layer "F.Cu") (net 25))
 (segment (start 141.6431 111.8616) (end 143.692775 109.811925) (width 0.3048) (layer "F.Cu") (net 25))
 (segment (start 137.1981 111.8616) (end 141.6431 111.8616) (width 0.3048) (layer "F.Cu") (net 25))
 (segment (start 134.5311 116.4336) (end 134.6581 116.3066) (width 0.3048) (layer "F.Cu") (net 25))
 (segment (start 131.9911 116.4336) (end 131.9911 114.5286) (width 0.3048) (layer "F.Cu") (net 24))
 (segment (start 141.273731 111.0996) (end 143.12709 109.246241) (width 0.3048) (layer "F.Cu") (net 24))
 (segment (start 135.4201 111.0996) (end 141.273731 111.0996) (width 0.3048) (layer "F.Cu") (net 24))
 (segment (start 131.9911 114.5286) (end 135.4201 111.0996) (width 0.3048) (layer "F.Cu") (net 24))
 (segment (start 129.5781 116.3066) (end 129.5781 114.4016) (width 0.3048) (layer "F.Cu") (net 23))
 (segment (start 133.6421 110.3376) (end 140.904356 110.3376) (width 0.3048) (layer "F.Cu") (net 23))
 (segment (start 129.5781 114.4016) (end 133.6421 110.3376) (width 0.3048) (layer "F.Cu") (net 23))
 (segment (start 129.4511 116.4336) (end 129.5781 116.3066) (width 0.3048) (layer "F.Cu") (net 23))
 (segment (start 140.904356 110.3376) (end 142.561403 108.680554) (width 0.3048) (layer "F.Cu") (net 23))
 (segment (start 126.9111 114.5286) (end 131.8641 109.5756) (width 0.3048) (layer "F.Cu") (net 22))
 (segment (start 140.534987 109.5756) (end 141.995718 108.114869) (width 0.3048) (layer "F.Cu") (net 22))
 (segment (start 131.8641 109.5756) (end 140.534987 109.5756) (width 0.3048) (layer "F.Cu") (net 22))
 (segment (start 126.9111 116.4336) (end 126.9111 114.5286) (width 0.3048) (layer "F.Cu") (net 22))
 (segment (start 130.0861 108.8136) (end 140.165618 108.8136) (width 0.3048) (layer "F.Cu") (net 21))
 (segment (start 140.165618 108.8136) (end 141.430034 107.549185) (width 0.3048) (layer "F.Cu") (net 21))
 (segment (start 124.3711 116.4336) (end 124.3711 114.5286) (width 0.3048) (layer "F.Cu") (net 21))
 (segment (start 124.3711 114.5286) (end 130.0861 108.8136) (width 0.3048) (layer "F.Cu") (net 21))
 (segment (start 131.9911 95.4786) (end 136.1821 99.6696) (width 0.3048) (layer "F.Cu") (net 17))
 (segment (start 131.9911 93.5736) (end 131.9911 95.4786) (width 0.3048) (layer "F.Cu") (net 17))
 (segment (start 140.904356 99.6696) (end 142.561403 101.326647) (width 0.3048) (layer "F.Cu") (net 17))
 (segment (start 136.1821 99.6696) (end 140.904356 99.6696) (width 0.3048) (layer "F.Cu") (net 17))
 (segment (start 140.165618 101.1936) (end 141.430034 102.458016) (width 0.3048) (layer "F.Cu") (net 19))
 (segment (start 126.9111 95.4786) (end 132.6261 101.1936) (width 0.3048) (layer "F.Cu") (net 19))
 (segment (start 126.9111 93.5736) (end 126.9111 95.4786) (width 0.3048) (layer "F.Cu") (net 19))
 (segment (start 132.6261 101.1936) (end 140.165618 101.1936) (width 0.3048) (layer "F.Cu") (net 19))
 (segment (start 139.6111 94.982232) (end 144.258459 99.629591) (width 0.3048) (layer "F.Cu") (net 14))
 (segment (start 139.6111 93.5736) (end 139.6111 94.982232) (width 0.3048) (layer "F.Cu") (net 14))
 (segment (start 130.8481 101.9556) (end 139.796243 101.9556) (width 0.3048) (layer "F.Cu") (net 20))
 (segment (start 124.3711 95.4786) (end 130.8481 101.9556) (width 0.3048) (layer "F.Cu") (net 20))
 (segment (start 139.796243 101.9556) (end 140.864346 103.023704) (width 0.3048) (layer "F.Cu") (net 20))
 (segment (start 124.3711 93.5736) (end 124.3711 95.4786) (width 0.3048) (layer "F.Cu") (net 20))
 (segment (start 140.534987 100.4316) (end 141.995718 101.892332) (width 0.3048) (layer "F.Cu") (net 18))
 (segment (start 129.4511 95.4786) (end 134.4041 100.4316) (width 0.3048) (layer "F.Cu") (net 18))
 (segment (start 129.4511 93.5736) (end 129.4511 95.4786) (width 0.3048) (layer "F.Cu") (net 18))
 (segment (start 134.4041 100.4316) (end 140.534987 100.4316) (width 0.3048) (layer "F.Cu") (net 18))
 (segment (start 137.0711 93.5736) (end 137.0711 95.4786) (width 0.3048) (layer "F.Cu") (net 15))
 (segment (start 139.7381 98.1456) (end 141.6431 98.1456) (width 0.3048) (layer "F.Cu") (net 15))
 (segment (start 141.6431 98.1456) (end 143.692775 100.195275) (width 0.3048) (layer "F.Cu") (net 15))
 (segment (start 137.0711 95.4786) (end 139.7381 98.1456) (width 0.3048) (layer "F.Cu") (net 15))
 (segment (start 145.267956 96.1136) (end 146.521203 97.366847) (width 0.3048) (layer "F.Cu") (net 13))
 (segment (start 142.1511 93.5736) (end 142.1511 95.4786) (width 0.3048) (layer "F.Cu") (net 13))
 (segment (start 142.1511 95.4786) (end 142.7861 96.1136) (width 0.3048) (layer "F.Cu") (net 13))
 (segment (start 142.7861 96.1136) (end 145.267956 96.1136) (width 0.3048) (layer "F.Cu") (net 13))
 (segment (start 141.273731 98.9076) (end 143.12709 100.76096) (width 0.3048) (layer "F.Cu") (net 16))
 (segment (start 134.5311 93.5736) (end 134.5311 95.4786) (width 0.3048) (layer "F.Cu") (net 16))
 (segment (start 137.9601 98.9076) (end 141.273731 98.9076) (width 0.3048) (layer "F.Cu") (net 16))
 (segment (start 134.5311 95.4786) (end 137.9601 98.9076) (width 0.3048) (layer "F.Cu") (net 16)))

